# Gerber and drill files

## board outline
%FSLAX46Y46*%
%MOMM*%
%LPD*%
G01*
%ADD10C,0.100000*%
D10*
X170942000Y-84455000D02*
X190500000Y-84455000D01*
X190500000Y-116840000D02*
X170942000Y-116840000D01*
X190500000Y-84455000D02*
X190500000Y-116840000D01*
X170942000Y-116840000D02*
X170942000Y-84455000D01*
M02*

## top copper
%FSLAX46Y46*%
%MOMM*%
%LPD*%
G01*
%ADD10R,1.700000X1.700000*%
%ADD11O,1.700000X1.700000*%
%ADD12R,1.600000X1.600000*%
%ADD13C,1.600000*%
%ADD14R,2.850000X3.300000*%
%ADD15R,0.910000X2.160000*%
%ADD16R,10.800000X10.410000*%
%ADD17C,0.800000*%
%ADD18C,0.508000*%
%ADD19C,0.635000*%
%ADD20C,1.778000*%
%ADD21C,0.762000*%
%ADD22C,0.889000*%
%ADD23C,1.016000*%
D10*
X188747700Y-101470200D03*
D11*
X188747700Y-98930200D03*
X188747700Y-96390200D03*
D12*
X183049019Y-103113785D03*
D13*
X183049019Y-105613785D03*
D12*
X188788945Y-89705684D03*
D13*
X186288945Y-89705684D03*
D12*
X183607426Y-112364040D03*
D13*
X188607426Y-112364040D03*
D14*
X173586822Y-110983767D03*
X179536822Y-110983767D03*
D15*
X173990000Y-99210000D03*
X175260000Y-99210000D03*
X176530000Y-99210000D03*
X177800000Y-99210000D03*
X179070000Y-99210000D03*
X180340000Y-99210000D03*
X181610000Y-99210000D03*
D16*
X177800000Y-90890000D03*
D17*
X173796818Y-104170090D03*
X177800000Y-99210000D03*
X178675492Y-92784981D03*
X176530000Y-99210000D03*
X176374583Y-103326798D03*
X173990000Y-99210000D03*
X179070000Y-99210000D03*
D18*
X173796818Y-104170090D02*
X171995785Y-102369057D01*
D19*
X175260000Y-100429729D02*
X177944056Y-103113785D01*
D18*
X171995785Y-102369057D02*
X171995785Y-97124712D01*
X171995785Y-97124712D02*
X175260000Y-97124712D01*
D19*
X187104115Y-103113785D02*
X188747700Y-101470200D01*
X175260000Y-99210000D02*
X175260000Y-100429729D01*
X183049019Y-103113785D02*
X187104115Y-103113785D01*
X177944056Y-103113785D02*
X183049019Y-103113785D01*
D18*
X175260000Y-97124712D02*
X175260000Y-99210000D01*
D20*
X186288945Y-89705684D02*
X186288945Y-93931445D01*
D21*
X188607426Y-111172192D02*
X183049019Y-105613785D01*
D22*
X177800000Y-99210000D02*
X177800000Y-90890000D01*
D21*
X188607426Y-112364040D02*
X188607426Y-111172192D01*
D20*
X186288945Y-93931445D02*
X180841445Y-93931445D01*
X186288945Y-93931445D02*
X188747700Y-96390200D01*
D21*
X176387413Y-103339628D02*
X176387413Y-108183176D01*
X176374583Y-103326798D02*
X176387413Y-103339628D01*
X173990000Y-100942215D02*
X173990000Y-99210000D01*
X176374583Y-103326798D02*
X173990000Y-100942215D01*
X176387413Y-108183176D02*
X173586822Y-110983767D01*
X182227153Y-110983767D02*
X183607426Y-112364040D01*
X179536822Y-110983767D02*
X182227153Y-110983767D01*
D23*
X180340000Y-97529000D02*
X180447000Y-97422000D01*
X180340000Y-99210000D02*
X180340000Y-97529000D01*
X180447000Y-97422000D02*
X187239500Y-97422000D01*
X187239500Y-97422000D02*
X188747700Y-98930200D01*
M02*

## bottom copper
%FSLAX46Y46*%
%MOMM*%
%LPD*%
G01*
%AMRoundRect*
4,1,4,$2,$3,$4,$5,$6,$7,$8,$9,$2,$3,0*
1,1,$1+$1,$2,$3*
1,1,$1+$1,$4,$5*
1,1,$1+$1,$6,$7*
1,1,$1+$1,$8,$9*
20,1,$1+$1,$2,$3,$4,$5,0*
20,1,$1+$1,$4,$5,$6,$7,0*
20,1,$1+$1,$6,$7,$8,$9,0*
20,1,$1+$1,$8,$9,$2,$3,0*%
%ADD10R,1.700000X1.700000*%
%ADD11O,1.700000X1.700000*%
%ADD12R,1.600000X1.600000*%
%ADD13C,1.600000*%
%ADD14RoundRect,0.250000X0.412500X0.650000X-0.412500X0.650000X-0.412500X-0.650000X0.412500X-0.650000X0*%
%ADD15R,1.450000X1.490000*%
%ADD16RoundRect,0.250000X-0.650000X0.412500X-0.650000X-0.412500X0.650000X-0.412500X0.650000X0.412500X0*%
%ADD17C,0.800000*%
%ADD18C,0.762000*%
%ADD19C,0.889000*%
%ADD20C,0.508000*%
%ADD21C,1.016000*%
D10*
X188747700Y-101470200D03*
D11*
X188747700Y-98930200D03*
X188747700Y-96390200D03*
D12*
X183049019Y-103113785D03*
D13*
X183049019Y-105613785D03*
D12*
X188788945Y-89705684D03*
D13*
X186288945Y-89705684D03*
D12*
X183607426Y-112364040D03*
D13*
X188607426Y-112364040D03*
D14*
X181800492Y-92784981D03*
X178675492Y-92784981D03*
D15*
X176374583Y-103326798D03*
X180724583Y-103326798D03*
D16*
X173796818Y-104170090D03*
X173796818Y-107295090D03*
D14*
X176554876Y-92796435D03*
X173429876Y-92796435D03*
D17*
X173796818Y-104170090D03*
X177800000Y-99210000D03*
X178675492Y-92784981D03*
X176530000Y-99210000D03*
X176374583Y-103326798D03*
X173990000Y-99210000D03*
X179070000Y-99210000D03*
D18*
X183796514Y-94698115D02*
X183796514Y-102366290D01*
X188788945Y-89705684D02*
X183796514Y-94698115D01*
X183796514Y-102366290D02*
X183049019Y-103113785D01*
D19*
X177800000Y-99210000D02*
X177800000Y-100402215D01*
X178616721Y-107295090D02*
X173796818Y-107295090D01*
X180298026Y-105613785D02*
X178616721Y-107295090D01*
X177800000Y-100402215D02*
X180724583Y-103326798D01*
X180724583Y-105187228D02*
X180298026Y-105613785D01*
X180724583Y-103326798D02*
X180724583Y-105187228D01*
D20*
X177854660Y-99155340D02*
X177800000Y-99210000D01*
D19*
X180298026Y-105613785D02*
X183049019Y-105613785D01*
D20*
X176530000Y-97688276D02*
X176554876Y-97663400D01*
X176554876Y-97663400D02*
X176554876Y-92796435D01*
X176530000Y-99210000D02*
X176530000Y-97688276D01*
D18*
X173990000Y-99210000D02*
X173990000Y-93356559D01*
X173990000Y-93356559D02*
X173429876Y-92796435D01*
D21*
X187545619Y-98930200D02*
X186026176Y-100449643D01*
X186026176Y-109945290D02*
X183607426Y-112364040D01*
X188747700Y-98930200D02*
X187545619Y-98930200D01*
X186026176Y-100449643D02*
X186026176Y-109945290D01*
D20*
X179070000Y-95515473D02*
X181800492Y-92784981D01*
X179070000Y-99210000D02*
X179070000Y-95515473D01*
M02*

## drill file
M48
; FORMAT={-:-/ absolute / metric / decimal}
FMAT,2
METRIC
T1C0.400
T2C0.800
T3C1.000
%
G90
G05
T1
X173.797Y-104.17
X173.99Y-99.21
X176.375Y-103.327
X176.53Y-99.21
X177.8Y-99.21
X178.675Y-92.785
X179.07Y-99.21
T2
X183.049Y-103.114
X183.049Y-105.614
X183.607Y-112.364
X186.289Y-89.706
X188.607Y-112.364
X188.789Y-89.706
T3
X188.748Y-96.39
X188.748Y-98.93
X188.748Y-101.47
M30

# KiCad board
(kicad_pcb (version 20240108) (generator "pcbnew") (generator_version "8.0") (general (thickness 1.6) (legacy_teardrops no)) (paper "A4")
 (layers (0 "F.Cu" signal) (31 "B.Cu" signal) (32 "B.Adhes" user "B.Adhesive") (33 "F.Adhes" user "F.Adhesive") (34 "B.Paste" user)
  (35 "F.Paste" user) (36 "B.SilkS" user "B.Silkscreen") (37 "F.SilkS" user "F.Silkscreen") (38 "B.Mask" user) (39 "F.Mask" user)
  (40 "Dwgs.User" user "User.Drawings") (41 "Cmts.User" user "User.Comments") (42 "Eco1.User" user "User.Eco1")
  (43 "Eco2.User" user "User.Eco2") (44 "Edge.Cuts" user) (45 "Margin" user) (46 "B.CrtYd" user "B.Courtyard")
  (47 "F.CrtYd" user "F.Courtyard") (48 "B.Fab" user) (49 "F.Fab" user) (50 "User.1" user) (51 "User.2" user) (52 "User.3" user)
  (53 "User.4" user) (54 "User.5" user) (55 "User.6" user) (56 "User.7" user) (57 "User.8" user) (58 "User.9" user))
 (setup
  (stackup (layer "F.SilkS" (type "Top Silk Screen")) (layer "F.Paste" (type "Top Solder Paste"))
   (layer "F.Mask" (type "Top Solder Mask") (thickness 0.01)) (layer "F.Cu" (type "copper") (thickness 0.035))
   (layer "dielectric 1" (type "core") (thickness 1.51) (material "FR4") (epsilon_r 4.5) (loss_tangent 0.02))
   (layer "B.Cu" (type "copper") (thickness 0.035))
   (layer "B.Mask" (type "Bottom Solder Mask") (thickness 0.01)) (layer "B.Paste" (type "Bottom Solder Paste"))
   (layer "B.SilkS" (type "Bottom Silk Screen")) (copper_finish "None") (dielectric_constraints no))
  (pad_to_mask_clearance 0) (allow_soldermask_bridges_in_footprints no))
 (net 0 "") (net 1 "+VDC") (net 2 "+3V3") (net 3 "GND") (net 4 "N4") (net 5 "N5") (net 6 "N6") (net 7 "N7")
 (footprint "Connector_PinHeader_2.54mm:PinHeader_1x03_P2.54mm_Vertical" (layer "F.Cu") (at 188.7477 101.4702 180)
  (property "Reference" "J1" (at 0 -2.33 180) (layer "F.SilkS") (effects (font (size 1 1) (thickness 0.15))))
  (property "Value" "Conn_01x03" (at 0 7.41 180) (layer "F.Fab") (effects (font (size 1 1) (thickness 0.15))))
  (pad "1" thru_hole rect (at 0 0 180) (size 1.7 1.7) (drill 1) (layers "*.Cu" "*.Mask") (remove_unused_layers no) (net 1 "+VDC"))
  (pad "2" thru_hole oval (at 0 2.54 180) (size 1.7 1.7) (drill 1) (layers "*.Cu" "*.Mask") (remove_unused_layers no) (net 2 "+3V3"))
  (pad "3" thru_hole oval (at 0 5.08 180) (size 1.7 1.7) (drill 1) (layers "*.Cu" "*.Mask") (remove_unused_layers no) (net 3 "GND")))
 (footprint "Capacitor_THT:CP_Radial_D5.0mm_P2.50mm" (layer "F.Cu") (at 183.049019 103.113785 -90)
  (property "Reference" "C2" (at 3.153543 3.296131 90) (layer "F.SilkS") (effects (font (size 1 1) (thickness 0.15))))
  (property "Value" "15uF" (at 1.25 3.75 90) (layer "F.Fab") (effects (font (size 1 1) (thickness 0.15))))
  (pad "1" thru_hole rect (at 0 0 270) (size 1.6 1.6) (drill 0.8) (layers "*.Cu" "*.Mask") (remove_unused_layers no) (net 1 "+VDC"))
  (pad "2" thru_hole circle (at 2.5 0 270) (size 1.6 1.6) (drill 0.8) (layers "*.Cu" "*.Mask") (remove_unused_layers no) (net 3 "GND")))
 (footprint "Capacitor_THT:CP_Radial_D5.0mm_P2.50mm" (layer "F.Cu") (at 188.788945 89.705684 180)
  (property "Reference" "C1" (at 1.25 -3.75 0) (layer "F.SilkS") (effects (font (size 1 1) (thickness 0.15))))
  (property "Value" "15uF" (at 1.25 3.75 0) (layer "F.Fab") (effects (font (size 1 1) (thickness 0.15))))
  (pad "1" thru_hole rect (at 0 0 180) (size 1.6 1.6) (drill 0.8) (layers "*.Cu" "*.Mask") (remove_unused_layers no) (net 1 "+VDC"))
  (pad "2" thru_hole circle (at 2.5 0 180) (size 1.6 1.6) (drill 0.8) (layers "*.Cu" "*.Mask") (remove_unused_layers no) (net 3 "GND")))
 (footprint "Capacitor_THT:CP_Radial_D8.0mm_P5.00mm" (layer "F.Cu") (at 183.607426 112.36404)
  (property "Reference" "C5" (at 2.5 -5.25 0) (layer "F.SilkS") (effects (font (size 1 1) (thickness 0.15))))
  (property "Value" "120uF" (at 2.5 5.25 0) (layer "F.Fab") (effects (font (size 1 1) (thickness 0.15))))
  (pad "1" thru_hole rect (at 0 0) (size 1.6 1.6) (drill 0.8) (layers "*.Cu" "*.Mask") (remove_unused_layers no) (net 2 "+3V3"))
  (pad "2" thru_hole circle (at 5 0) (size 1.6 1.6) (drill 0.8) (layers "*.Cu" "*.Mask") (remove_unused_layers no) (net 3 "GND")))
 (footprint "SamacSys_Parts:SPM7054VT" (layer "F.Cu") (at 176.561822 110.983767)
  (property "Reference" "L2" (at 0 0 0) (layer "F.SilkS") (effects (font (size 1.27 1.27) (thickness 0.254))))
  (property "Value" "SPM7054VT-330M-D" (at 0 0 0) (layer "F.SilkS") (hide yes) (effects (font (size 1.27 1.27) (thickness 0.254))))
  (pad "1" smd rect (at -2.975 0) (size 2.85 3.3) (layers "F.Cu" "F.Paste" "F.Mask") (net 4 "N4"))
  (pad "2" smd rect (at 2.975 0) (size 2.85 3.3) (layers "F.Cu" "F.Paste" "F.Mask") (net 2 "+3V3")))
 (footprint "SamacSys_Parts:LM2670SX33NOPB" (layer "F.Cu") (at 177.8 91.44 -90)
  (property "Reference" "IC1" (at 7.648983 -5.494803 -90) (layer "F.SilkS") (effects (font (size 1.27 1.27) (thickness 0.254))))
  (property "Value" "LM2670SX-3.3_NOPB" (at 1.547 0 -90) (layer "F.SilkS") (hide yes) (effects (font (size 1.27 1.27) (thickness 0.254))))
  (pad "1" smd rect (at 7.77 3.81) (size 0.91 2.16) (layers "F.Cu" "F.Paste" "F.Mask") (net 4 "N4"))
  (pad "2" smd rect (at 7.77 2.54) (size 0.91 2.16) (layers "F.Cu" "F.Paste" "F.Mask") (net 1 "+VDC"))
  (pad "3" smd rect (at 7.77 1.27) (size 0.91 2.16) (layers "F.Cu" "F.Paste" "F.Mask") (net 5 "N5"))
  (pad "4" smd rect (at 7.77 0) (size 0.91 2.16) (layers "F.Cu" "F.Paste" "F.Mask") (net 3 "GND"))
  (pad "5" smd rect (at 7.77 -1.27) (size 0.91 2.16) (layers "F.Cu" "F.Paste" "F.Mask") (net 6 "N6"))
  (pad "6" smd rect (at 7.77 -2.54) (size 0.91 2.16) (layers "F.Cu" "F.Paste" "F.Mask") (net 2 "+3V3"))
  (pad "7" smd rect (at 7.77 -3.81) (size 0.91 2.16) (layers "F.Cu" "F.Paste" "F.Mask") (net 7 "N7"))
  (pad "8" smd rect (at -0.55 0 270) (size 10.41 10.8) (layers "F.Cu" "F.Paste" "F.Mask") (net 3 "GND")))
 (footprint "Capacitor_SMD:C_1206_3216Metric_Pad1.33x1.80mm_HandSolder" (layer "B.Cu") (at 180.237992 92.784981 180)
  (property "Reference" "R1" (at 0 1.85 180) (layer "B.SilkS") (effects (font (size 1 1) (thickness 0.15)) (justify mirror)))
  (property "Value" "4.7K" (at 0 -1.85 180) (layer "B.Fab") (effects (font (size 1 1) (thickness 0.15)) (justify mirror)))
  (pad "1" smd roundrect (at -1.5625 0 180) (size 1.325 1.8) (layers "B.Cu" "B.Paste" "B.Mask") (roundrect_rratio 0.188679) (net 6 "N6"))
  (pad "2" smd roundrect (at 1.5625 0 180) (size 1.325 1.8) (layers "B.Cu" "B.Paste" "B.Mask") (roundrect_rratio 0.188679) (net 3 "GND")))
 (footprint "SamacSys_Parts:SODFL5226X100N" (layer "B.Cu") (at 178.549583 103.326798)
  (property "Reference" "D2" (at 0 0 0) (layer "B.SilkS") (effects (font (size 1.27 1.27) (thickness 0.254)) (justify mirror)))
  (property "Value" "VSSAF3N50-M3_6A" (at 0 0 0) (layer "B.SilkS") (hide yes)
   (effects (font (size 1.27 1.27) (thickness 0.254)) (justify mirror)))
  (pad "1" smd rect (at -2.175 0) (size 1.45 1.49) (layers "B.Cu" "B.Paste" "B.Mask") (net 4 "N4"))
  (pad "2" smd rect (at 2.175 0) (size 1.45 1.49) (layers "B.Cu" "B.Paste" "B.Mask") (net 3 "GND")))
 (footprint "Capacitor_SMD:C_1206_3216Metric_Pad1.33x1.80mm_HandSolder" (layer "B.Cu") (at 173.796818 105.73259 -90)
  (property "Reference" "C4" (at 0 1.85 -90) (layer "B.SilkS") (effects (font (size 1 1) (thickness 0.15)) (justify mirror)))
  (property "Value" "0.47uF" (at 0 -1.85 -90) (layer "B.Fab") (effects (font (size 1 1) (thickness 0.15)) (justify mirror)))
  (pad "1" smd roundrect (at -1.5625 0 270) (size 1.325 1.8) (layers "B.Cu" "B.Paste" "B.Mask") (roundrect_rratio 0.188679) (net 1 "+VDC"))
  (pad "2" smd roundrect (at 1.5625 0 270) (size 1.325 1.8) (layers "B.Cu" "B.Paste" "B.Mask") (roundrect_rratio 0.188679) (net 3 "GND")))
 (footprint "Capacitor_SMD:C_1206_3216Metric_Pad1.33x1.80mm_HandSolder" (layer "B.Cu") (at 174.992376 92.796435 180)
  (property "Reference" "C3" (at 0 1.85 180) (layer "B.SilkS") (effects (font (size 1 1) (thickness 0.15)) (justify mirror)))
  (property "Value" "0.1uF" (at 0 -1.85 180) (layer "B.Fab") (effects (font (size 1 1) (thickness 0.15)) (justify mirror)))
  (pad "1" smd roundrect (at -1.5625 0 180) (size 1.325 1.8) (layers "B.Cu" "B.Paste" "B.Mask") (roundrect_rratio 0.188679) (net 5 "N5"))
  (pad "2" smd roundrect (at 1.5625 0 180) (size 1.325 1.8) (layers "B.Cu" "B.Paste" "B.Mask") (roundrect_rratio 0.188679) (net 4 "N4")))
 (gr_line (start 170.942 84.455) (end 190.5 84.455) (stroke (width 0.1) (type solid)) (layer "Edge.Cuts"))
 (gr_line (start 190.5 116.84) (end 170.942 116.84) (stroke (width 0.1) (type default)) (layer "Edge.Cuts"))
 (gr_line (start 190.5 84.455) (end 190.5 116.84) (stroke (width 0.1) (type default)) (layer "Edge.Cuts"))
 (gr_line (start 170.942 116.84) (end 170.942 84.455) (stroke (width 0.1) (type solid)) (layer "Edge.Cuts"))
 (segment (start 173.796818 104.17009) (end 171.995785 102.369057) (width 0.508) (layer "F.Cu") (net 1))
 (segment (start 175.26 100.429729) (end 177.944056 103.113785) (width 0.635) (layer "F.Cu") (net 1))
 (segment (start 171.995785 102.369057) (end 171.995785 97.124712) (width 0.508) (layer "F.Cu") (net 1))
 (segment (start 171.995785 97.124712) (end 175.26 97.124712) (width 0.508) (layer "F.Cu") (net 1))
 (segment (start 187.104115 103.113785) (end 188.7477 101.4702) (width 0.635) (layer "F.Cu") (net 1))
 (segment (start 175.26 99.21) (end 175.26 100.429729) (width 0.635) (layer "F.Cu") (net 1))
 (segment (start 183.049019 103.113785) (end 187.104115 103.113785) (width 0.635) (layer "F.Cu") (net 1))
 (segment (start 177.944056 103.113785) (end 183.049019 103.113785) (width 0.635) (layer "F.Cu") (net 1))
 (segment (start 175.26 97.124712) (end 175.26 99.21) (width 0.508) (layer "F.Cu") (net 1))
 (via (at 173.796818 104.17009) (size 0.8) (drill 0.4) (layers "F.Cu" "B.Cu") (free yes) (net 1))
 (segment (start 183.796514 94.698115) (end 183.796514 102.36629) (width 0.762) (layer "B.Cu") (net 1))
 (segment (start 188.788945 89.705684) (end 183.796514 94.698115) (width 0.762) (layer "B.Cu") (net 1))
 (segment (start 183.796514 102.36629) (end 183.049019 103.113785) (width 0.762) (layer "B.Cu") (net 1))
 (segment (start 186.288945 89.705684) (end 186.288945 93.931445) (width 1.778) (layer "F.Cu") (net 3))
 (segment (start 188.607426 111.172192) (end 183.049019 105.613785) (width 0.762) (layer "F.Cu") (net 3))
 (segment (start 177.8 99.21) (end 177.8 90.89) (width 0.889) (layer "F.Cu") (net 3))
 (segment (start 188.607426 112.36404) (end 188.607426 111.172192) (width 0.762) (layer "F.Cu") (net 3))
 (segment (start 186.288945 93.931445) (end 180.841445 93.931445) (width 1.778) (layer "F.Cu") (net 3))
 (segment (start 186.288945 93.931445) (end 188.7477 96.3902) (width 1.778) (layer "F.Cu") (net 3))
 (via (at 177.8 99.21) (size 0.8) (drill 0.4) (layers "F.Cu" "B.Cu") (free yes) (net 3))
 (via (at 178.675492 92.784981) (size 0.8) (drill 0.4) (layers "F.Cu" "B.Cu") (free yes) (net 3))
 (segment (start 177.8 99.21) (end 177.8 100.402215) (width 0.889) (layer "B.Cu") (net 3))
 (segment (start 178.616721 107.29509) (end 173.796818 107.29509) (width 0.889) (layer "B.Cu") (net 3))
 (segment (start 180.298026 105.613785) (end 178.616721 107.29509) (width 0.889) (layer "B.Cu") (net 3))
 (segment (start 177.8 100.402215) (end 180.724583 103.326798) (width 0.889) (layer "B.Cu") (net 3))
 (segment (start 180.724583 105.187228) (end 180.298026 105.613785) (width 0.889) (layer "B.Cu") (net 3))
 (segment (start 180.724583 103.326798) (end 180.724583 105.187228) (width 0.889) (layer "B.Cu") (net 3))
 (segment (start 177.85466 99.15534) (end 177.8 99.21) (width 0.508) (layer "B.Cu") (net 3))
 (segment (start 180.298026 105.613785) (end 183.049019 105.613785) (width 0.889) (layer "B.Cu") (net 3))
 (via (at 176.53 99.21) (size 0.8) (drill 0.4) (layers "F.Cu" "B.Cu") (free yes) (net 5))
 (segment (start 176.53 97.688276) (end 176.554876 97.6634) (width 0.508) (layer "B.Cu") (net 5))
 (segment (start 176.554876 97.6634) (end 176.554876 92.796435) (width 0.508) (layer "B.Cu") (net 5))
 (segment (start 176.53 99.21) (end 176.53 97.688276) (width 0.508) (layer "B.Cu") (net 5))
 (segment (start 176.387413 103.339628) (end 176.387413 108.183176) (width 0.762) (layer "F.Cu") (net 4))
 (segment (start 176.374583 103.326798) (end 176.387413 103.339628) (width 0.762) (layer "F.Cu") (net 4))
 (segment (start 173.99 100.942215) (end 173.99 99.21) (width 0.762) (layer "F.Cu") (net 4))
 (segment (start 176.374583 103.326798) (end 173.99 100.942215) (width 0.762) (layer "F.Cu") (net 4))
 (segment (start 176.387413 108.183176) (end 173.586822 110.983767) (width 0.762) (layer "F.Cu") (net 4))
 (via (at 176.374583 103.326798) (size 0.8) (drill 0.4) (layers "F.Cu" "B.Cu") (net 4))
 (via (at 173.99 99.21) (size 0.8) (drill 0.4) (layers "F.Cu" "B.Cu") (free yes) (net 4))
 (segment (start 173.99 99.21) (end 173.99 93.356559) (width 0.762) (layer "B.Cu") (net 4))
 (segment (start 173.99 93.356559) (end 173.429876 92.796435) (width 0.762) (layer "B.Cu") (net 4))
 (segment (start 182.227153 110.983767) (end 183.607426 112.36404) (width 0.762) (layer "F.Cu") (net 2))
 (segment (start 179.536822 110.983767) (end 182.227153 110.983767) (width 0.762) (layer "F.Cu") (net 2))
 (segment (start 180.34 97.529) (end 180.447 97.422) (width 1.016) (layer "F.Cu") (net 2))
 (segment (start 180.34 99.21) (end 180.34 97.529) (width 1.016) (layer "F.Cu") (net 2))
 (segment (start 180.447 97.422) (end 187.2395 97.422) (width 1.016) (layer "F.Cu") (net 2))
 (segment (start 187.2395 97.422) (end 188.7477 98.9302) (width 1.016) (layer "F.Cu") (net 2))
 (segment (start 187.545619 98.9302) (end 186.026176 100.449643) (width 1.016) (layer "B.Cu") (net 2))
 (segment (start 186.026176 109.94529) (end 183.607426 112.36404) (width 1.016) (layer "B.Cu") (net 2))
 (segment (start 188.7477 98.9302) (end 187.545619 98.9302) (width 1.016) (layer "B.Cu") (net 2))
 (segment (start 186.026176 100.449643) (end 186.026176 109.94529) (width 1.016) (layer "B.Cu") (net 2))
 (via (at 179.07 99.21) (size 0.8) (drill 0.4) (layers "F.Cu" "B.Cu") (free yes) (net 6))
 (segment (start 179.07 95.515473) (end 181.800492 92.784981) (width 0.508) (layer "B.Cu") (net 6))
 (segment (start 179.07 99.21) (end 179.07 95.515473) (width 0.508) (layer "B.Cu") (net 6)))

